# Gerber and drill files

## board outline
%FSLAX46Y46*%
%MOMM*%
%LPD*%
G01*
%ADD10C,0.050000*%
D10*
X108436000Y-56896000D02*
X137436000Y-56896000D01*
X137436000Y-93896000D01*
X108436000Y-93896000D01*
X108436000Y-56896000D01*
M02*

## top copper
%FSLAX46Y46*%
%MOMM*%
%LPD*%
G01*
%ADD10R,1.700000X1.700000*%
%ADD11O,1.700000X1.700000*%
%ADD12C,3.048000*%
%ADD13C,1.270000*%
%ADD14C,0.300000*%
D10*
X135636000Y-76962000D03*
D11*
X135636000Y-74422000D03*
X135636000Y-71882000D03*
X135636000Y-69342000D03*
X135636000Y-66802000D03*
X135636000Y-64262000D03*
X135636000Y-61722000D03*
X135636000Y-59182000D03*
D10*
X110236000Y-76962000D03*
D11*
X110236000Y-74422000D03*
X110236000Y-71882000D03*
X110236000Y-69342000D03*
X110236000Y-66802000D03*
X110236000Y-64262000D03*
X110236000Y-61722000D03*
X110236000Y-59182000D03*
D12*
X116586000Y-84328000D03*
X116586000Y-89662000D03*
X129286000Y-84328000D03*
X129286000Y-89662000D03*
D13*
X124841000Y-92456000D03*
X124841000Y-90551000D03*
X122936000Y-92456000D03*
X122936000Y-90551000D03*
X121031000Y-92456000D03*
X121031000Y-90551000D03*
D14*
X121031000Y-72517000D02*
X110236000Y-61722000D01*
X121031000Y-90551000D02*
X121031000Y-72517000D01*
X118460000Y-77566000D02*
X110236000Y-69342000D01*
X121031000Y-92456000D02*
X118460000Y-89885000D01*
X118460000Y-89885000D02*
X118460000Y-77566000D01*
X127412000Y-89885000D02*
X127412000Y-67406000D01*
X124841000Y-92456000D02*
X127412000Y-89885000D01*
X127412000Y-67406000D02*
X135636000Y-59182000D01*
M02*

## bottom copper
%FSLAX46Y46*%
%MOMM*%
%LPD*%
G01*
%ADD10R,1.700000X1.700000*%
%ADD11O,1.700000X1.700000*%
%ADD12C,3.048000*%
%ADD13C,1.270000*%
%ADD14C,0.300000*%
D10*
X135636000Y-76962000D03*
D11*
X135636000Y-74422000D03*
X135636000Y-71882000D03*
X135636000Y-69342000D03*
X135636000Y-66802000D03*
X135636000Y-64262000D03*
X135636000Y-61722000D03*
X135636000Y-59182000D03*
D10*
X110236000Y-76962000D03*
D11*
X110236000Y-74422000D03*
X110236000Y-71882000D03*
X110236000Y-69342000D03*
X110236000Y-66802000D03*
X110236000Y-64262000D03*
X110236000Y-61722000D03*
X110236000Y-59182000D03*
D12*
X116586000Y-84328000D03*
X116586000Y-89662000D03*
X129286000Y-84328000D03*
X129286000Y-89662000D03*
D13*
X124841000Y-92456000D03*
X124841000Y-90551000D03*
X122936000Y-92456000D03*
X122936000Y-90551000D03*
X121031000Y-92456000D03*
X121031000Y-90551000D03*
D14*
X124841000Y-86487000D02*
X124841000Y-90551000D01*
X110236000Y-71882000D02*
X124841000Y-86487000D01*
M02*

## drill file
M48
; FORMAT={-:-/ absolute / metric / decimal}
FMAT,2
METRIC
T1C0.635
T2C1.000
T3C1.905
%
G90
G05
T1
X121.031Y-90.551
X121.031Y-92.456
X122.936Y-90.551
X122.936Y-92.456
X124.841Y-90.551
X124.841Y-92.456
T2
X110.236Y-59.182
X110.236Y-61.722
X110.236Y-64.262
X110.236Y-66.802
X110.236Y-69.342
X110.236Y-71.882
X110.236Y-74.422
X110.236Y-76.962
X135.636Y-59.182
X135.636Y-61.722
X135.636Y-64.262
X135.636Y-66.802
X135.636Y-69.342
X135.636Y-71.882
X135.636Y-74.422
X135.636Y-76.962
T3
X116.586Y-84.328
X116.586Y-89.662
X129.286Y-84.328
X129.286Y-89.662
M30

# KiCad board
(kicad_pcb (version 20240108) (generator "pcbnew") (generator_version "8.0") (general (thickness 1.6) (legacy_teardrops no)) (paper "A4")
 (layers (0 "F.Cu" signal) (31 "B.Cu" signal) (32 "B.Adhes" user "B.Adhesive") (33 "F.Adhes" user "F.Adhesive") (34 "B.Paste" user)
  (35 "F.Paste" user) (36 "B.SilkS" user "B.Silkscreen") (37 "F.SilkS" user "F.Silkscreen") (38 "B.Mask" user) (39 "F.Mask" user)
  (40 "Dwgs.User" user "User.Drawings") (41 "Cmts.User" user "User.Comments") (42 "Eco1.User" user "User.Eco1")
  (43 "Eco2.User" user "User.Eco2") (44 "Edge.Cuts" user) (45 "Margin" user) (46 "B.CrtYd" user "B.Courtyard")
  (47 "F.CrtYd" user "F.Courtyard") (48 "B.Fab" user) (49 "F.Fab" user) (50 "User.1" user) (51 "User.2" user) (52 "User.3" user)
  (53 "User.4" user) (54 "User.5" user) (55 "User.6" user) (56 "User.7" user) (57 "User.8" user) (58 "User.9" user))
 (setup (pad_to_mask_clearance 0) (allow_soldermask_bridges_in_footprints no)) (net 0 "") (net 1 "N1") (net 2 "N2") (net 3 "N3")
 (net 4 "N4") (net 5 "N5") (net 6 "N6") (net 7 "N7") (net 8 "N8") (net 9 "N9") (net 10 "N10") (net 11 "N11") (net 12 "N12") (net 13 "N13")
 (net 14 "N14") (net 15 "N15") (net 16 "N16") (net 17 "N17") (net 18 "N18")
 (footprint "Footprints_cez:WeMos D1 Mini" (layer "F.Cu") (at 122.682 85.471 180)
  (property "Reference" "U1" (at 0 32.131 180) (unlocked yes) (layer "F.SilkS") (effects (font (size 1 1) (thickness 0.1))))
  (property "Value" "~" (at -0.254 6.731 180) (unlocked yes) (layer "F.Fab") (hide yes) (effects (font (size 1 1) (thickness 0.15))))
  (pad "1" thru_hole rect (at -12.954 8.509 180) (size 1.7 1.7) (drill 1) (layers "*.Cu" "*.Mask") (remove_unused_layers no) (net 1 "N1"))
  (pad "2" thru_hole oval (at -12.954 11.049 180) (size 1.7 1.7) (drill 1) (layers "*.Cu" "*.Mask") (remove_unused_layers no) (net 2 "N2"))
  (pad "3" thru_hole oval (at -12.954 13.589 180) (size 1.7 1.7) (drill 1) (layers "*.Cu" "*.Mask") (remove_unused_layers no) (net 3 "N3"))
  (pad "4" thru_hole oval (at -12.954 16.129 180) (size 1.7 1.7) (drill 1) (layers "*.Cu" "*.Mask") (remove_unused_layers no) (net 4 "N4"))
  (pad "5" thru_hole oval (at -12.954 18.669 180) (size 1.7 1.7) (drill 1) (layers "*.Cu" "*.Mask") (remove_unused_layers no) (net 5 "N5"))
  (pad "6" thru_hole oval (at -12.954 21.209 180) (size 1.7 1.7) (drill 1) (layers "*.Cu" "*.Mask") (remove_unused_layers no) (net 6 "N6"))
  (pad "7" thru_hole oval (at -12.954 23.749 180) (size 1.7 1.7) (drill 1) (layers "*.Cu" "*.Mask") (remove_unused_layers no) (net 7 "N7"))
  (pad "8" thru_hole oval (at -12.954 26.289 180) (size 1.7 1.7) (drill 1) (layers "*.Cu" "*.Mask") (remove_unused_layers no) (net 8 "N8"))
  (pad "9" thru_hole rect (at 12.446 8.509 180) (size 1.7 1.7) (drill 1) (layers "*.Cu" "*.Mask") (remove_unused_layers no) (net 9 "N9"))
  (pad "10" thru_hole oval (at 12.446 11.049 180) (size 1.7 1.7) (drill 1) (layers "*.Cu" "*.Mask") (remove_unused_layers no) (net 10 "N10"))
  (pad "11" thru_hole oval (at 12.446 13.589 180) (size 1.7 1.7) (drill 1) (layers "*.Cu" "*.Mask") (remove_unused_layers no) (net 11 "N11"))
  (pad "12" thru_hole oval (at 12.446 16.129 180) (size 1.7 1.7) (drill 1) (layers "*.Cu" "*.Mask") (remove_unused_layers no) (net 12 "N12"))
  (pad "13" thru_hole oval (at 12.446 18.669 180) (size 1.7 1.7) (drill 1) (layers "*.Cu" "*.Mask") (remove_unused_layers no) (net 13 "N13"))
  (pad "14" thru_hole oval (at 12.446 21.209 180) (size 1.7 1.7) (drill 1) (layers "*.Cu" "*.Mask") (remove_unused_layers no) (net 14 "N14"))
  (pad "15" thru_hole oval (at 12.446 23.749 180) (size 1.7 1.7) (drill 1) (layers "*.Cu" "*.Mask") (remove_unused_layers no) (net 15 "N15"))
  (pad "16" thru_hole oval (at 12.446 26.289 180) (size 1.7 1.7) (drill 1) (layers "*.Cu" "*.Mask") (remove_unused_layers no) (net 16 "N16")))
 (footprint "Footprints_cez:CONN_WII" (layer "F.Cu") (at 122.936 86.868)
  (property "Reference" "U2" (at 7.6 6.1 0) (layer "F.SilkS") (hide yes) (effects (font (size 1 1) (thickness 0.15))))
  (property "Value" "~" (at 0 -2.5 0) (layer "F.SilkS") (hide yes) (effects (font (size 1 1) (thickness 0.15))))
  (pad "" thru_hole circle (at -6.35 -2.54) (size 3.048 3.048) (drill 1.905) (layers "*.Cu" "*.Mask") (remove_unused_layers no))
  (pad "" thru_hole circle (at -6.35 2.794) (size 3.048 3.048) (drill 1.905) (layers "*.Cu" "*.Mask") (remove_unused_layers no))
  (pad "" thru_hole circle (at 6.35 -2.54) (size 3.048 3.048) (drill 1.905) (layers "*.Cu" "*.Mask") (remove_unused_layers no))
  (pad "" thru_hole circle (at 6.35 2.794) (size 3.048 3.048) (drill 1.905) (layers "*.Cu" "*.Mask") (remove_unused_layers no))
  (pad "1" thru_hole circle (at 1.905 5.588) (size 1.27 1.27) (drill 0.635) (layers "*.Cu" "*.Mask") (remove_unused_layers no) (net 8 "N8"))
  (pad "2" thru_hole circle (at 1.905 3.683) (size 1.27 1.27) (drill 0.635) (layers "*.Cu" "*.Mask") (remove_unused_layers no)
   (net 11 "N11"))
  (pad "3" thru_hole circle (at 0 5.588) (size 1.27 1.27) (drill 0.635) (layers "*.Cu" "*.Mask") (remove_unused_layers no) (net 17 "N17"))
  (pad "4" thru_hole circle (at 0 3.683) (size 1.27 1.27) (drill 0.635) (layers "*.Cu" "*.Mask") (remove_unused_layers no) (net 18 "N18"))
  (pad "5" thru_hole circle (at -1.905 5.588) (size 1.27 1.27) (drill 0.635) (layers "*.Cu" "*.Mask") (remove_unused_layers no)
   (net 12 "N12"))
  (pad "6" thru_hole circle (at -1.905 3.683) (size 1.27 1.27) (drill 0.635) (layers "*.Cu" "*.Mask") (remove_unused_layers no)
   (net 15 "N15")))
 (gr_rect (start 108.436 56.896) (end 137.436 93.896) (stroke (width 0.05) (type default)) (fill none) (layer "Edge.Cuts"))
 (segment (start 121.031 72.517) (end 110.236 61.722) (width 0.3) (layer "F.Cu") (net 15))
 (segment (start 121.031 90.551) (end 121.031 72.517) (width 0.3) (layer "F.Cu") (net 15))
 (segment (start 124.841 86.487) (end 124.841 90.551) (width 0.3) (layer "B.Cu") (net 11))
 (segment (start 110.236 71.882) (end 124.841 86.487) (width 0.3) (layer "B.Cu") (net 11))
 (segment (start 118.46 77.566) (end 110.236 69.342) (width 0.3) (layer "F.Cu") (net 12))
 (segment (start 121.031 92.456) (end 118.46 89.885) (width 0.3) (layer "F.Cu") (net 12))
 (segment (start 118.46 89.885) (end 118.46 77.566) (width 0.3) (layer "F.Cu") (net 12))
 (segment (start 127.412 89.885) (end 127.412 67.406) (width 0.3) (layer "F.Cu") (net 8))
 (segment (start 124.841 92.456) (end 127.412 89.885) (width 0.3) (layer "F.Cu") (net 8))
 (segment (start 127.412 67.406) (end 135.636 59.182) (width 0.3) (layer "F.Cu") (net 8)))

